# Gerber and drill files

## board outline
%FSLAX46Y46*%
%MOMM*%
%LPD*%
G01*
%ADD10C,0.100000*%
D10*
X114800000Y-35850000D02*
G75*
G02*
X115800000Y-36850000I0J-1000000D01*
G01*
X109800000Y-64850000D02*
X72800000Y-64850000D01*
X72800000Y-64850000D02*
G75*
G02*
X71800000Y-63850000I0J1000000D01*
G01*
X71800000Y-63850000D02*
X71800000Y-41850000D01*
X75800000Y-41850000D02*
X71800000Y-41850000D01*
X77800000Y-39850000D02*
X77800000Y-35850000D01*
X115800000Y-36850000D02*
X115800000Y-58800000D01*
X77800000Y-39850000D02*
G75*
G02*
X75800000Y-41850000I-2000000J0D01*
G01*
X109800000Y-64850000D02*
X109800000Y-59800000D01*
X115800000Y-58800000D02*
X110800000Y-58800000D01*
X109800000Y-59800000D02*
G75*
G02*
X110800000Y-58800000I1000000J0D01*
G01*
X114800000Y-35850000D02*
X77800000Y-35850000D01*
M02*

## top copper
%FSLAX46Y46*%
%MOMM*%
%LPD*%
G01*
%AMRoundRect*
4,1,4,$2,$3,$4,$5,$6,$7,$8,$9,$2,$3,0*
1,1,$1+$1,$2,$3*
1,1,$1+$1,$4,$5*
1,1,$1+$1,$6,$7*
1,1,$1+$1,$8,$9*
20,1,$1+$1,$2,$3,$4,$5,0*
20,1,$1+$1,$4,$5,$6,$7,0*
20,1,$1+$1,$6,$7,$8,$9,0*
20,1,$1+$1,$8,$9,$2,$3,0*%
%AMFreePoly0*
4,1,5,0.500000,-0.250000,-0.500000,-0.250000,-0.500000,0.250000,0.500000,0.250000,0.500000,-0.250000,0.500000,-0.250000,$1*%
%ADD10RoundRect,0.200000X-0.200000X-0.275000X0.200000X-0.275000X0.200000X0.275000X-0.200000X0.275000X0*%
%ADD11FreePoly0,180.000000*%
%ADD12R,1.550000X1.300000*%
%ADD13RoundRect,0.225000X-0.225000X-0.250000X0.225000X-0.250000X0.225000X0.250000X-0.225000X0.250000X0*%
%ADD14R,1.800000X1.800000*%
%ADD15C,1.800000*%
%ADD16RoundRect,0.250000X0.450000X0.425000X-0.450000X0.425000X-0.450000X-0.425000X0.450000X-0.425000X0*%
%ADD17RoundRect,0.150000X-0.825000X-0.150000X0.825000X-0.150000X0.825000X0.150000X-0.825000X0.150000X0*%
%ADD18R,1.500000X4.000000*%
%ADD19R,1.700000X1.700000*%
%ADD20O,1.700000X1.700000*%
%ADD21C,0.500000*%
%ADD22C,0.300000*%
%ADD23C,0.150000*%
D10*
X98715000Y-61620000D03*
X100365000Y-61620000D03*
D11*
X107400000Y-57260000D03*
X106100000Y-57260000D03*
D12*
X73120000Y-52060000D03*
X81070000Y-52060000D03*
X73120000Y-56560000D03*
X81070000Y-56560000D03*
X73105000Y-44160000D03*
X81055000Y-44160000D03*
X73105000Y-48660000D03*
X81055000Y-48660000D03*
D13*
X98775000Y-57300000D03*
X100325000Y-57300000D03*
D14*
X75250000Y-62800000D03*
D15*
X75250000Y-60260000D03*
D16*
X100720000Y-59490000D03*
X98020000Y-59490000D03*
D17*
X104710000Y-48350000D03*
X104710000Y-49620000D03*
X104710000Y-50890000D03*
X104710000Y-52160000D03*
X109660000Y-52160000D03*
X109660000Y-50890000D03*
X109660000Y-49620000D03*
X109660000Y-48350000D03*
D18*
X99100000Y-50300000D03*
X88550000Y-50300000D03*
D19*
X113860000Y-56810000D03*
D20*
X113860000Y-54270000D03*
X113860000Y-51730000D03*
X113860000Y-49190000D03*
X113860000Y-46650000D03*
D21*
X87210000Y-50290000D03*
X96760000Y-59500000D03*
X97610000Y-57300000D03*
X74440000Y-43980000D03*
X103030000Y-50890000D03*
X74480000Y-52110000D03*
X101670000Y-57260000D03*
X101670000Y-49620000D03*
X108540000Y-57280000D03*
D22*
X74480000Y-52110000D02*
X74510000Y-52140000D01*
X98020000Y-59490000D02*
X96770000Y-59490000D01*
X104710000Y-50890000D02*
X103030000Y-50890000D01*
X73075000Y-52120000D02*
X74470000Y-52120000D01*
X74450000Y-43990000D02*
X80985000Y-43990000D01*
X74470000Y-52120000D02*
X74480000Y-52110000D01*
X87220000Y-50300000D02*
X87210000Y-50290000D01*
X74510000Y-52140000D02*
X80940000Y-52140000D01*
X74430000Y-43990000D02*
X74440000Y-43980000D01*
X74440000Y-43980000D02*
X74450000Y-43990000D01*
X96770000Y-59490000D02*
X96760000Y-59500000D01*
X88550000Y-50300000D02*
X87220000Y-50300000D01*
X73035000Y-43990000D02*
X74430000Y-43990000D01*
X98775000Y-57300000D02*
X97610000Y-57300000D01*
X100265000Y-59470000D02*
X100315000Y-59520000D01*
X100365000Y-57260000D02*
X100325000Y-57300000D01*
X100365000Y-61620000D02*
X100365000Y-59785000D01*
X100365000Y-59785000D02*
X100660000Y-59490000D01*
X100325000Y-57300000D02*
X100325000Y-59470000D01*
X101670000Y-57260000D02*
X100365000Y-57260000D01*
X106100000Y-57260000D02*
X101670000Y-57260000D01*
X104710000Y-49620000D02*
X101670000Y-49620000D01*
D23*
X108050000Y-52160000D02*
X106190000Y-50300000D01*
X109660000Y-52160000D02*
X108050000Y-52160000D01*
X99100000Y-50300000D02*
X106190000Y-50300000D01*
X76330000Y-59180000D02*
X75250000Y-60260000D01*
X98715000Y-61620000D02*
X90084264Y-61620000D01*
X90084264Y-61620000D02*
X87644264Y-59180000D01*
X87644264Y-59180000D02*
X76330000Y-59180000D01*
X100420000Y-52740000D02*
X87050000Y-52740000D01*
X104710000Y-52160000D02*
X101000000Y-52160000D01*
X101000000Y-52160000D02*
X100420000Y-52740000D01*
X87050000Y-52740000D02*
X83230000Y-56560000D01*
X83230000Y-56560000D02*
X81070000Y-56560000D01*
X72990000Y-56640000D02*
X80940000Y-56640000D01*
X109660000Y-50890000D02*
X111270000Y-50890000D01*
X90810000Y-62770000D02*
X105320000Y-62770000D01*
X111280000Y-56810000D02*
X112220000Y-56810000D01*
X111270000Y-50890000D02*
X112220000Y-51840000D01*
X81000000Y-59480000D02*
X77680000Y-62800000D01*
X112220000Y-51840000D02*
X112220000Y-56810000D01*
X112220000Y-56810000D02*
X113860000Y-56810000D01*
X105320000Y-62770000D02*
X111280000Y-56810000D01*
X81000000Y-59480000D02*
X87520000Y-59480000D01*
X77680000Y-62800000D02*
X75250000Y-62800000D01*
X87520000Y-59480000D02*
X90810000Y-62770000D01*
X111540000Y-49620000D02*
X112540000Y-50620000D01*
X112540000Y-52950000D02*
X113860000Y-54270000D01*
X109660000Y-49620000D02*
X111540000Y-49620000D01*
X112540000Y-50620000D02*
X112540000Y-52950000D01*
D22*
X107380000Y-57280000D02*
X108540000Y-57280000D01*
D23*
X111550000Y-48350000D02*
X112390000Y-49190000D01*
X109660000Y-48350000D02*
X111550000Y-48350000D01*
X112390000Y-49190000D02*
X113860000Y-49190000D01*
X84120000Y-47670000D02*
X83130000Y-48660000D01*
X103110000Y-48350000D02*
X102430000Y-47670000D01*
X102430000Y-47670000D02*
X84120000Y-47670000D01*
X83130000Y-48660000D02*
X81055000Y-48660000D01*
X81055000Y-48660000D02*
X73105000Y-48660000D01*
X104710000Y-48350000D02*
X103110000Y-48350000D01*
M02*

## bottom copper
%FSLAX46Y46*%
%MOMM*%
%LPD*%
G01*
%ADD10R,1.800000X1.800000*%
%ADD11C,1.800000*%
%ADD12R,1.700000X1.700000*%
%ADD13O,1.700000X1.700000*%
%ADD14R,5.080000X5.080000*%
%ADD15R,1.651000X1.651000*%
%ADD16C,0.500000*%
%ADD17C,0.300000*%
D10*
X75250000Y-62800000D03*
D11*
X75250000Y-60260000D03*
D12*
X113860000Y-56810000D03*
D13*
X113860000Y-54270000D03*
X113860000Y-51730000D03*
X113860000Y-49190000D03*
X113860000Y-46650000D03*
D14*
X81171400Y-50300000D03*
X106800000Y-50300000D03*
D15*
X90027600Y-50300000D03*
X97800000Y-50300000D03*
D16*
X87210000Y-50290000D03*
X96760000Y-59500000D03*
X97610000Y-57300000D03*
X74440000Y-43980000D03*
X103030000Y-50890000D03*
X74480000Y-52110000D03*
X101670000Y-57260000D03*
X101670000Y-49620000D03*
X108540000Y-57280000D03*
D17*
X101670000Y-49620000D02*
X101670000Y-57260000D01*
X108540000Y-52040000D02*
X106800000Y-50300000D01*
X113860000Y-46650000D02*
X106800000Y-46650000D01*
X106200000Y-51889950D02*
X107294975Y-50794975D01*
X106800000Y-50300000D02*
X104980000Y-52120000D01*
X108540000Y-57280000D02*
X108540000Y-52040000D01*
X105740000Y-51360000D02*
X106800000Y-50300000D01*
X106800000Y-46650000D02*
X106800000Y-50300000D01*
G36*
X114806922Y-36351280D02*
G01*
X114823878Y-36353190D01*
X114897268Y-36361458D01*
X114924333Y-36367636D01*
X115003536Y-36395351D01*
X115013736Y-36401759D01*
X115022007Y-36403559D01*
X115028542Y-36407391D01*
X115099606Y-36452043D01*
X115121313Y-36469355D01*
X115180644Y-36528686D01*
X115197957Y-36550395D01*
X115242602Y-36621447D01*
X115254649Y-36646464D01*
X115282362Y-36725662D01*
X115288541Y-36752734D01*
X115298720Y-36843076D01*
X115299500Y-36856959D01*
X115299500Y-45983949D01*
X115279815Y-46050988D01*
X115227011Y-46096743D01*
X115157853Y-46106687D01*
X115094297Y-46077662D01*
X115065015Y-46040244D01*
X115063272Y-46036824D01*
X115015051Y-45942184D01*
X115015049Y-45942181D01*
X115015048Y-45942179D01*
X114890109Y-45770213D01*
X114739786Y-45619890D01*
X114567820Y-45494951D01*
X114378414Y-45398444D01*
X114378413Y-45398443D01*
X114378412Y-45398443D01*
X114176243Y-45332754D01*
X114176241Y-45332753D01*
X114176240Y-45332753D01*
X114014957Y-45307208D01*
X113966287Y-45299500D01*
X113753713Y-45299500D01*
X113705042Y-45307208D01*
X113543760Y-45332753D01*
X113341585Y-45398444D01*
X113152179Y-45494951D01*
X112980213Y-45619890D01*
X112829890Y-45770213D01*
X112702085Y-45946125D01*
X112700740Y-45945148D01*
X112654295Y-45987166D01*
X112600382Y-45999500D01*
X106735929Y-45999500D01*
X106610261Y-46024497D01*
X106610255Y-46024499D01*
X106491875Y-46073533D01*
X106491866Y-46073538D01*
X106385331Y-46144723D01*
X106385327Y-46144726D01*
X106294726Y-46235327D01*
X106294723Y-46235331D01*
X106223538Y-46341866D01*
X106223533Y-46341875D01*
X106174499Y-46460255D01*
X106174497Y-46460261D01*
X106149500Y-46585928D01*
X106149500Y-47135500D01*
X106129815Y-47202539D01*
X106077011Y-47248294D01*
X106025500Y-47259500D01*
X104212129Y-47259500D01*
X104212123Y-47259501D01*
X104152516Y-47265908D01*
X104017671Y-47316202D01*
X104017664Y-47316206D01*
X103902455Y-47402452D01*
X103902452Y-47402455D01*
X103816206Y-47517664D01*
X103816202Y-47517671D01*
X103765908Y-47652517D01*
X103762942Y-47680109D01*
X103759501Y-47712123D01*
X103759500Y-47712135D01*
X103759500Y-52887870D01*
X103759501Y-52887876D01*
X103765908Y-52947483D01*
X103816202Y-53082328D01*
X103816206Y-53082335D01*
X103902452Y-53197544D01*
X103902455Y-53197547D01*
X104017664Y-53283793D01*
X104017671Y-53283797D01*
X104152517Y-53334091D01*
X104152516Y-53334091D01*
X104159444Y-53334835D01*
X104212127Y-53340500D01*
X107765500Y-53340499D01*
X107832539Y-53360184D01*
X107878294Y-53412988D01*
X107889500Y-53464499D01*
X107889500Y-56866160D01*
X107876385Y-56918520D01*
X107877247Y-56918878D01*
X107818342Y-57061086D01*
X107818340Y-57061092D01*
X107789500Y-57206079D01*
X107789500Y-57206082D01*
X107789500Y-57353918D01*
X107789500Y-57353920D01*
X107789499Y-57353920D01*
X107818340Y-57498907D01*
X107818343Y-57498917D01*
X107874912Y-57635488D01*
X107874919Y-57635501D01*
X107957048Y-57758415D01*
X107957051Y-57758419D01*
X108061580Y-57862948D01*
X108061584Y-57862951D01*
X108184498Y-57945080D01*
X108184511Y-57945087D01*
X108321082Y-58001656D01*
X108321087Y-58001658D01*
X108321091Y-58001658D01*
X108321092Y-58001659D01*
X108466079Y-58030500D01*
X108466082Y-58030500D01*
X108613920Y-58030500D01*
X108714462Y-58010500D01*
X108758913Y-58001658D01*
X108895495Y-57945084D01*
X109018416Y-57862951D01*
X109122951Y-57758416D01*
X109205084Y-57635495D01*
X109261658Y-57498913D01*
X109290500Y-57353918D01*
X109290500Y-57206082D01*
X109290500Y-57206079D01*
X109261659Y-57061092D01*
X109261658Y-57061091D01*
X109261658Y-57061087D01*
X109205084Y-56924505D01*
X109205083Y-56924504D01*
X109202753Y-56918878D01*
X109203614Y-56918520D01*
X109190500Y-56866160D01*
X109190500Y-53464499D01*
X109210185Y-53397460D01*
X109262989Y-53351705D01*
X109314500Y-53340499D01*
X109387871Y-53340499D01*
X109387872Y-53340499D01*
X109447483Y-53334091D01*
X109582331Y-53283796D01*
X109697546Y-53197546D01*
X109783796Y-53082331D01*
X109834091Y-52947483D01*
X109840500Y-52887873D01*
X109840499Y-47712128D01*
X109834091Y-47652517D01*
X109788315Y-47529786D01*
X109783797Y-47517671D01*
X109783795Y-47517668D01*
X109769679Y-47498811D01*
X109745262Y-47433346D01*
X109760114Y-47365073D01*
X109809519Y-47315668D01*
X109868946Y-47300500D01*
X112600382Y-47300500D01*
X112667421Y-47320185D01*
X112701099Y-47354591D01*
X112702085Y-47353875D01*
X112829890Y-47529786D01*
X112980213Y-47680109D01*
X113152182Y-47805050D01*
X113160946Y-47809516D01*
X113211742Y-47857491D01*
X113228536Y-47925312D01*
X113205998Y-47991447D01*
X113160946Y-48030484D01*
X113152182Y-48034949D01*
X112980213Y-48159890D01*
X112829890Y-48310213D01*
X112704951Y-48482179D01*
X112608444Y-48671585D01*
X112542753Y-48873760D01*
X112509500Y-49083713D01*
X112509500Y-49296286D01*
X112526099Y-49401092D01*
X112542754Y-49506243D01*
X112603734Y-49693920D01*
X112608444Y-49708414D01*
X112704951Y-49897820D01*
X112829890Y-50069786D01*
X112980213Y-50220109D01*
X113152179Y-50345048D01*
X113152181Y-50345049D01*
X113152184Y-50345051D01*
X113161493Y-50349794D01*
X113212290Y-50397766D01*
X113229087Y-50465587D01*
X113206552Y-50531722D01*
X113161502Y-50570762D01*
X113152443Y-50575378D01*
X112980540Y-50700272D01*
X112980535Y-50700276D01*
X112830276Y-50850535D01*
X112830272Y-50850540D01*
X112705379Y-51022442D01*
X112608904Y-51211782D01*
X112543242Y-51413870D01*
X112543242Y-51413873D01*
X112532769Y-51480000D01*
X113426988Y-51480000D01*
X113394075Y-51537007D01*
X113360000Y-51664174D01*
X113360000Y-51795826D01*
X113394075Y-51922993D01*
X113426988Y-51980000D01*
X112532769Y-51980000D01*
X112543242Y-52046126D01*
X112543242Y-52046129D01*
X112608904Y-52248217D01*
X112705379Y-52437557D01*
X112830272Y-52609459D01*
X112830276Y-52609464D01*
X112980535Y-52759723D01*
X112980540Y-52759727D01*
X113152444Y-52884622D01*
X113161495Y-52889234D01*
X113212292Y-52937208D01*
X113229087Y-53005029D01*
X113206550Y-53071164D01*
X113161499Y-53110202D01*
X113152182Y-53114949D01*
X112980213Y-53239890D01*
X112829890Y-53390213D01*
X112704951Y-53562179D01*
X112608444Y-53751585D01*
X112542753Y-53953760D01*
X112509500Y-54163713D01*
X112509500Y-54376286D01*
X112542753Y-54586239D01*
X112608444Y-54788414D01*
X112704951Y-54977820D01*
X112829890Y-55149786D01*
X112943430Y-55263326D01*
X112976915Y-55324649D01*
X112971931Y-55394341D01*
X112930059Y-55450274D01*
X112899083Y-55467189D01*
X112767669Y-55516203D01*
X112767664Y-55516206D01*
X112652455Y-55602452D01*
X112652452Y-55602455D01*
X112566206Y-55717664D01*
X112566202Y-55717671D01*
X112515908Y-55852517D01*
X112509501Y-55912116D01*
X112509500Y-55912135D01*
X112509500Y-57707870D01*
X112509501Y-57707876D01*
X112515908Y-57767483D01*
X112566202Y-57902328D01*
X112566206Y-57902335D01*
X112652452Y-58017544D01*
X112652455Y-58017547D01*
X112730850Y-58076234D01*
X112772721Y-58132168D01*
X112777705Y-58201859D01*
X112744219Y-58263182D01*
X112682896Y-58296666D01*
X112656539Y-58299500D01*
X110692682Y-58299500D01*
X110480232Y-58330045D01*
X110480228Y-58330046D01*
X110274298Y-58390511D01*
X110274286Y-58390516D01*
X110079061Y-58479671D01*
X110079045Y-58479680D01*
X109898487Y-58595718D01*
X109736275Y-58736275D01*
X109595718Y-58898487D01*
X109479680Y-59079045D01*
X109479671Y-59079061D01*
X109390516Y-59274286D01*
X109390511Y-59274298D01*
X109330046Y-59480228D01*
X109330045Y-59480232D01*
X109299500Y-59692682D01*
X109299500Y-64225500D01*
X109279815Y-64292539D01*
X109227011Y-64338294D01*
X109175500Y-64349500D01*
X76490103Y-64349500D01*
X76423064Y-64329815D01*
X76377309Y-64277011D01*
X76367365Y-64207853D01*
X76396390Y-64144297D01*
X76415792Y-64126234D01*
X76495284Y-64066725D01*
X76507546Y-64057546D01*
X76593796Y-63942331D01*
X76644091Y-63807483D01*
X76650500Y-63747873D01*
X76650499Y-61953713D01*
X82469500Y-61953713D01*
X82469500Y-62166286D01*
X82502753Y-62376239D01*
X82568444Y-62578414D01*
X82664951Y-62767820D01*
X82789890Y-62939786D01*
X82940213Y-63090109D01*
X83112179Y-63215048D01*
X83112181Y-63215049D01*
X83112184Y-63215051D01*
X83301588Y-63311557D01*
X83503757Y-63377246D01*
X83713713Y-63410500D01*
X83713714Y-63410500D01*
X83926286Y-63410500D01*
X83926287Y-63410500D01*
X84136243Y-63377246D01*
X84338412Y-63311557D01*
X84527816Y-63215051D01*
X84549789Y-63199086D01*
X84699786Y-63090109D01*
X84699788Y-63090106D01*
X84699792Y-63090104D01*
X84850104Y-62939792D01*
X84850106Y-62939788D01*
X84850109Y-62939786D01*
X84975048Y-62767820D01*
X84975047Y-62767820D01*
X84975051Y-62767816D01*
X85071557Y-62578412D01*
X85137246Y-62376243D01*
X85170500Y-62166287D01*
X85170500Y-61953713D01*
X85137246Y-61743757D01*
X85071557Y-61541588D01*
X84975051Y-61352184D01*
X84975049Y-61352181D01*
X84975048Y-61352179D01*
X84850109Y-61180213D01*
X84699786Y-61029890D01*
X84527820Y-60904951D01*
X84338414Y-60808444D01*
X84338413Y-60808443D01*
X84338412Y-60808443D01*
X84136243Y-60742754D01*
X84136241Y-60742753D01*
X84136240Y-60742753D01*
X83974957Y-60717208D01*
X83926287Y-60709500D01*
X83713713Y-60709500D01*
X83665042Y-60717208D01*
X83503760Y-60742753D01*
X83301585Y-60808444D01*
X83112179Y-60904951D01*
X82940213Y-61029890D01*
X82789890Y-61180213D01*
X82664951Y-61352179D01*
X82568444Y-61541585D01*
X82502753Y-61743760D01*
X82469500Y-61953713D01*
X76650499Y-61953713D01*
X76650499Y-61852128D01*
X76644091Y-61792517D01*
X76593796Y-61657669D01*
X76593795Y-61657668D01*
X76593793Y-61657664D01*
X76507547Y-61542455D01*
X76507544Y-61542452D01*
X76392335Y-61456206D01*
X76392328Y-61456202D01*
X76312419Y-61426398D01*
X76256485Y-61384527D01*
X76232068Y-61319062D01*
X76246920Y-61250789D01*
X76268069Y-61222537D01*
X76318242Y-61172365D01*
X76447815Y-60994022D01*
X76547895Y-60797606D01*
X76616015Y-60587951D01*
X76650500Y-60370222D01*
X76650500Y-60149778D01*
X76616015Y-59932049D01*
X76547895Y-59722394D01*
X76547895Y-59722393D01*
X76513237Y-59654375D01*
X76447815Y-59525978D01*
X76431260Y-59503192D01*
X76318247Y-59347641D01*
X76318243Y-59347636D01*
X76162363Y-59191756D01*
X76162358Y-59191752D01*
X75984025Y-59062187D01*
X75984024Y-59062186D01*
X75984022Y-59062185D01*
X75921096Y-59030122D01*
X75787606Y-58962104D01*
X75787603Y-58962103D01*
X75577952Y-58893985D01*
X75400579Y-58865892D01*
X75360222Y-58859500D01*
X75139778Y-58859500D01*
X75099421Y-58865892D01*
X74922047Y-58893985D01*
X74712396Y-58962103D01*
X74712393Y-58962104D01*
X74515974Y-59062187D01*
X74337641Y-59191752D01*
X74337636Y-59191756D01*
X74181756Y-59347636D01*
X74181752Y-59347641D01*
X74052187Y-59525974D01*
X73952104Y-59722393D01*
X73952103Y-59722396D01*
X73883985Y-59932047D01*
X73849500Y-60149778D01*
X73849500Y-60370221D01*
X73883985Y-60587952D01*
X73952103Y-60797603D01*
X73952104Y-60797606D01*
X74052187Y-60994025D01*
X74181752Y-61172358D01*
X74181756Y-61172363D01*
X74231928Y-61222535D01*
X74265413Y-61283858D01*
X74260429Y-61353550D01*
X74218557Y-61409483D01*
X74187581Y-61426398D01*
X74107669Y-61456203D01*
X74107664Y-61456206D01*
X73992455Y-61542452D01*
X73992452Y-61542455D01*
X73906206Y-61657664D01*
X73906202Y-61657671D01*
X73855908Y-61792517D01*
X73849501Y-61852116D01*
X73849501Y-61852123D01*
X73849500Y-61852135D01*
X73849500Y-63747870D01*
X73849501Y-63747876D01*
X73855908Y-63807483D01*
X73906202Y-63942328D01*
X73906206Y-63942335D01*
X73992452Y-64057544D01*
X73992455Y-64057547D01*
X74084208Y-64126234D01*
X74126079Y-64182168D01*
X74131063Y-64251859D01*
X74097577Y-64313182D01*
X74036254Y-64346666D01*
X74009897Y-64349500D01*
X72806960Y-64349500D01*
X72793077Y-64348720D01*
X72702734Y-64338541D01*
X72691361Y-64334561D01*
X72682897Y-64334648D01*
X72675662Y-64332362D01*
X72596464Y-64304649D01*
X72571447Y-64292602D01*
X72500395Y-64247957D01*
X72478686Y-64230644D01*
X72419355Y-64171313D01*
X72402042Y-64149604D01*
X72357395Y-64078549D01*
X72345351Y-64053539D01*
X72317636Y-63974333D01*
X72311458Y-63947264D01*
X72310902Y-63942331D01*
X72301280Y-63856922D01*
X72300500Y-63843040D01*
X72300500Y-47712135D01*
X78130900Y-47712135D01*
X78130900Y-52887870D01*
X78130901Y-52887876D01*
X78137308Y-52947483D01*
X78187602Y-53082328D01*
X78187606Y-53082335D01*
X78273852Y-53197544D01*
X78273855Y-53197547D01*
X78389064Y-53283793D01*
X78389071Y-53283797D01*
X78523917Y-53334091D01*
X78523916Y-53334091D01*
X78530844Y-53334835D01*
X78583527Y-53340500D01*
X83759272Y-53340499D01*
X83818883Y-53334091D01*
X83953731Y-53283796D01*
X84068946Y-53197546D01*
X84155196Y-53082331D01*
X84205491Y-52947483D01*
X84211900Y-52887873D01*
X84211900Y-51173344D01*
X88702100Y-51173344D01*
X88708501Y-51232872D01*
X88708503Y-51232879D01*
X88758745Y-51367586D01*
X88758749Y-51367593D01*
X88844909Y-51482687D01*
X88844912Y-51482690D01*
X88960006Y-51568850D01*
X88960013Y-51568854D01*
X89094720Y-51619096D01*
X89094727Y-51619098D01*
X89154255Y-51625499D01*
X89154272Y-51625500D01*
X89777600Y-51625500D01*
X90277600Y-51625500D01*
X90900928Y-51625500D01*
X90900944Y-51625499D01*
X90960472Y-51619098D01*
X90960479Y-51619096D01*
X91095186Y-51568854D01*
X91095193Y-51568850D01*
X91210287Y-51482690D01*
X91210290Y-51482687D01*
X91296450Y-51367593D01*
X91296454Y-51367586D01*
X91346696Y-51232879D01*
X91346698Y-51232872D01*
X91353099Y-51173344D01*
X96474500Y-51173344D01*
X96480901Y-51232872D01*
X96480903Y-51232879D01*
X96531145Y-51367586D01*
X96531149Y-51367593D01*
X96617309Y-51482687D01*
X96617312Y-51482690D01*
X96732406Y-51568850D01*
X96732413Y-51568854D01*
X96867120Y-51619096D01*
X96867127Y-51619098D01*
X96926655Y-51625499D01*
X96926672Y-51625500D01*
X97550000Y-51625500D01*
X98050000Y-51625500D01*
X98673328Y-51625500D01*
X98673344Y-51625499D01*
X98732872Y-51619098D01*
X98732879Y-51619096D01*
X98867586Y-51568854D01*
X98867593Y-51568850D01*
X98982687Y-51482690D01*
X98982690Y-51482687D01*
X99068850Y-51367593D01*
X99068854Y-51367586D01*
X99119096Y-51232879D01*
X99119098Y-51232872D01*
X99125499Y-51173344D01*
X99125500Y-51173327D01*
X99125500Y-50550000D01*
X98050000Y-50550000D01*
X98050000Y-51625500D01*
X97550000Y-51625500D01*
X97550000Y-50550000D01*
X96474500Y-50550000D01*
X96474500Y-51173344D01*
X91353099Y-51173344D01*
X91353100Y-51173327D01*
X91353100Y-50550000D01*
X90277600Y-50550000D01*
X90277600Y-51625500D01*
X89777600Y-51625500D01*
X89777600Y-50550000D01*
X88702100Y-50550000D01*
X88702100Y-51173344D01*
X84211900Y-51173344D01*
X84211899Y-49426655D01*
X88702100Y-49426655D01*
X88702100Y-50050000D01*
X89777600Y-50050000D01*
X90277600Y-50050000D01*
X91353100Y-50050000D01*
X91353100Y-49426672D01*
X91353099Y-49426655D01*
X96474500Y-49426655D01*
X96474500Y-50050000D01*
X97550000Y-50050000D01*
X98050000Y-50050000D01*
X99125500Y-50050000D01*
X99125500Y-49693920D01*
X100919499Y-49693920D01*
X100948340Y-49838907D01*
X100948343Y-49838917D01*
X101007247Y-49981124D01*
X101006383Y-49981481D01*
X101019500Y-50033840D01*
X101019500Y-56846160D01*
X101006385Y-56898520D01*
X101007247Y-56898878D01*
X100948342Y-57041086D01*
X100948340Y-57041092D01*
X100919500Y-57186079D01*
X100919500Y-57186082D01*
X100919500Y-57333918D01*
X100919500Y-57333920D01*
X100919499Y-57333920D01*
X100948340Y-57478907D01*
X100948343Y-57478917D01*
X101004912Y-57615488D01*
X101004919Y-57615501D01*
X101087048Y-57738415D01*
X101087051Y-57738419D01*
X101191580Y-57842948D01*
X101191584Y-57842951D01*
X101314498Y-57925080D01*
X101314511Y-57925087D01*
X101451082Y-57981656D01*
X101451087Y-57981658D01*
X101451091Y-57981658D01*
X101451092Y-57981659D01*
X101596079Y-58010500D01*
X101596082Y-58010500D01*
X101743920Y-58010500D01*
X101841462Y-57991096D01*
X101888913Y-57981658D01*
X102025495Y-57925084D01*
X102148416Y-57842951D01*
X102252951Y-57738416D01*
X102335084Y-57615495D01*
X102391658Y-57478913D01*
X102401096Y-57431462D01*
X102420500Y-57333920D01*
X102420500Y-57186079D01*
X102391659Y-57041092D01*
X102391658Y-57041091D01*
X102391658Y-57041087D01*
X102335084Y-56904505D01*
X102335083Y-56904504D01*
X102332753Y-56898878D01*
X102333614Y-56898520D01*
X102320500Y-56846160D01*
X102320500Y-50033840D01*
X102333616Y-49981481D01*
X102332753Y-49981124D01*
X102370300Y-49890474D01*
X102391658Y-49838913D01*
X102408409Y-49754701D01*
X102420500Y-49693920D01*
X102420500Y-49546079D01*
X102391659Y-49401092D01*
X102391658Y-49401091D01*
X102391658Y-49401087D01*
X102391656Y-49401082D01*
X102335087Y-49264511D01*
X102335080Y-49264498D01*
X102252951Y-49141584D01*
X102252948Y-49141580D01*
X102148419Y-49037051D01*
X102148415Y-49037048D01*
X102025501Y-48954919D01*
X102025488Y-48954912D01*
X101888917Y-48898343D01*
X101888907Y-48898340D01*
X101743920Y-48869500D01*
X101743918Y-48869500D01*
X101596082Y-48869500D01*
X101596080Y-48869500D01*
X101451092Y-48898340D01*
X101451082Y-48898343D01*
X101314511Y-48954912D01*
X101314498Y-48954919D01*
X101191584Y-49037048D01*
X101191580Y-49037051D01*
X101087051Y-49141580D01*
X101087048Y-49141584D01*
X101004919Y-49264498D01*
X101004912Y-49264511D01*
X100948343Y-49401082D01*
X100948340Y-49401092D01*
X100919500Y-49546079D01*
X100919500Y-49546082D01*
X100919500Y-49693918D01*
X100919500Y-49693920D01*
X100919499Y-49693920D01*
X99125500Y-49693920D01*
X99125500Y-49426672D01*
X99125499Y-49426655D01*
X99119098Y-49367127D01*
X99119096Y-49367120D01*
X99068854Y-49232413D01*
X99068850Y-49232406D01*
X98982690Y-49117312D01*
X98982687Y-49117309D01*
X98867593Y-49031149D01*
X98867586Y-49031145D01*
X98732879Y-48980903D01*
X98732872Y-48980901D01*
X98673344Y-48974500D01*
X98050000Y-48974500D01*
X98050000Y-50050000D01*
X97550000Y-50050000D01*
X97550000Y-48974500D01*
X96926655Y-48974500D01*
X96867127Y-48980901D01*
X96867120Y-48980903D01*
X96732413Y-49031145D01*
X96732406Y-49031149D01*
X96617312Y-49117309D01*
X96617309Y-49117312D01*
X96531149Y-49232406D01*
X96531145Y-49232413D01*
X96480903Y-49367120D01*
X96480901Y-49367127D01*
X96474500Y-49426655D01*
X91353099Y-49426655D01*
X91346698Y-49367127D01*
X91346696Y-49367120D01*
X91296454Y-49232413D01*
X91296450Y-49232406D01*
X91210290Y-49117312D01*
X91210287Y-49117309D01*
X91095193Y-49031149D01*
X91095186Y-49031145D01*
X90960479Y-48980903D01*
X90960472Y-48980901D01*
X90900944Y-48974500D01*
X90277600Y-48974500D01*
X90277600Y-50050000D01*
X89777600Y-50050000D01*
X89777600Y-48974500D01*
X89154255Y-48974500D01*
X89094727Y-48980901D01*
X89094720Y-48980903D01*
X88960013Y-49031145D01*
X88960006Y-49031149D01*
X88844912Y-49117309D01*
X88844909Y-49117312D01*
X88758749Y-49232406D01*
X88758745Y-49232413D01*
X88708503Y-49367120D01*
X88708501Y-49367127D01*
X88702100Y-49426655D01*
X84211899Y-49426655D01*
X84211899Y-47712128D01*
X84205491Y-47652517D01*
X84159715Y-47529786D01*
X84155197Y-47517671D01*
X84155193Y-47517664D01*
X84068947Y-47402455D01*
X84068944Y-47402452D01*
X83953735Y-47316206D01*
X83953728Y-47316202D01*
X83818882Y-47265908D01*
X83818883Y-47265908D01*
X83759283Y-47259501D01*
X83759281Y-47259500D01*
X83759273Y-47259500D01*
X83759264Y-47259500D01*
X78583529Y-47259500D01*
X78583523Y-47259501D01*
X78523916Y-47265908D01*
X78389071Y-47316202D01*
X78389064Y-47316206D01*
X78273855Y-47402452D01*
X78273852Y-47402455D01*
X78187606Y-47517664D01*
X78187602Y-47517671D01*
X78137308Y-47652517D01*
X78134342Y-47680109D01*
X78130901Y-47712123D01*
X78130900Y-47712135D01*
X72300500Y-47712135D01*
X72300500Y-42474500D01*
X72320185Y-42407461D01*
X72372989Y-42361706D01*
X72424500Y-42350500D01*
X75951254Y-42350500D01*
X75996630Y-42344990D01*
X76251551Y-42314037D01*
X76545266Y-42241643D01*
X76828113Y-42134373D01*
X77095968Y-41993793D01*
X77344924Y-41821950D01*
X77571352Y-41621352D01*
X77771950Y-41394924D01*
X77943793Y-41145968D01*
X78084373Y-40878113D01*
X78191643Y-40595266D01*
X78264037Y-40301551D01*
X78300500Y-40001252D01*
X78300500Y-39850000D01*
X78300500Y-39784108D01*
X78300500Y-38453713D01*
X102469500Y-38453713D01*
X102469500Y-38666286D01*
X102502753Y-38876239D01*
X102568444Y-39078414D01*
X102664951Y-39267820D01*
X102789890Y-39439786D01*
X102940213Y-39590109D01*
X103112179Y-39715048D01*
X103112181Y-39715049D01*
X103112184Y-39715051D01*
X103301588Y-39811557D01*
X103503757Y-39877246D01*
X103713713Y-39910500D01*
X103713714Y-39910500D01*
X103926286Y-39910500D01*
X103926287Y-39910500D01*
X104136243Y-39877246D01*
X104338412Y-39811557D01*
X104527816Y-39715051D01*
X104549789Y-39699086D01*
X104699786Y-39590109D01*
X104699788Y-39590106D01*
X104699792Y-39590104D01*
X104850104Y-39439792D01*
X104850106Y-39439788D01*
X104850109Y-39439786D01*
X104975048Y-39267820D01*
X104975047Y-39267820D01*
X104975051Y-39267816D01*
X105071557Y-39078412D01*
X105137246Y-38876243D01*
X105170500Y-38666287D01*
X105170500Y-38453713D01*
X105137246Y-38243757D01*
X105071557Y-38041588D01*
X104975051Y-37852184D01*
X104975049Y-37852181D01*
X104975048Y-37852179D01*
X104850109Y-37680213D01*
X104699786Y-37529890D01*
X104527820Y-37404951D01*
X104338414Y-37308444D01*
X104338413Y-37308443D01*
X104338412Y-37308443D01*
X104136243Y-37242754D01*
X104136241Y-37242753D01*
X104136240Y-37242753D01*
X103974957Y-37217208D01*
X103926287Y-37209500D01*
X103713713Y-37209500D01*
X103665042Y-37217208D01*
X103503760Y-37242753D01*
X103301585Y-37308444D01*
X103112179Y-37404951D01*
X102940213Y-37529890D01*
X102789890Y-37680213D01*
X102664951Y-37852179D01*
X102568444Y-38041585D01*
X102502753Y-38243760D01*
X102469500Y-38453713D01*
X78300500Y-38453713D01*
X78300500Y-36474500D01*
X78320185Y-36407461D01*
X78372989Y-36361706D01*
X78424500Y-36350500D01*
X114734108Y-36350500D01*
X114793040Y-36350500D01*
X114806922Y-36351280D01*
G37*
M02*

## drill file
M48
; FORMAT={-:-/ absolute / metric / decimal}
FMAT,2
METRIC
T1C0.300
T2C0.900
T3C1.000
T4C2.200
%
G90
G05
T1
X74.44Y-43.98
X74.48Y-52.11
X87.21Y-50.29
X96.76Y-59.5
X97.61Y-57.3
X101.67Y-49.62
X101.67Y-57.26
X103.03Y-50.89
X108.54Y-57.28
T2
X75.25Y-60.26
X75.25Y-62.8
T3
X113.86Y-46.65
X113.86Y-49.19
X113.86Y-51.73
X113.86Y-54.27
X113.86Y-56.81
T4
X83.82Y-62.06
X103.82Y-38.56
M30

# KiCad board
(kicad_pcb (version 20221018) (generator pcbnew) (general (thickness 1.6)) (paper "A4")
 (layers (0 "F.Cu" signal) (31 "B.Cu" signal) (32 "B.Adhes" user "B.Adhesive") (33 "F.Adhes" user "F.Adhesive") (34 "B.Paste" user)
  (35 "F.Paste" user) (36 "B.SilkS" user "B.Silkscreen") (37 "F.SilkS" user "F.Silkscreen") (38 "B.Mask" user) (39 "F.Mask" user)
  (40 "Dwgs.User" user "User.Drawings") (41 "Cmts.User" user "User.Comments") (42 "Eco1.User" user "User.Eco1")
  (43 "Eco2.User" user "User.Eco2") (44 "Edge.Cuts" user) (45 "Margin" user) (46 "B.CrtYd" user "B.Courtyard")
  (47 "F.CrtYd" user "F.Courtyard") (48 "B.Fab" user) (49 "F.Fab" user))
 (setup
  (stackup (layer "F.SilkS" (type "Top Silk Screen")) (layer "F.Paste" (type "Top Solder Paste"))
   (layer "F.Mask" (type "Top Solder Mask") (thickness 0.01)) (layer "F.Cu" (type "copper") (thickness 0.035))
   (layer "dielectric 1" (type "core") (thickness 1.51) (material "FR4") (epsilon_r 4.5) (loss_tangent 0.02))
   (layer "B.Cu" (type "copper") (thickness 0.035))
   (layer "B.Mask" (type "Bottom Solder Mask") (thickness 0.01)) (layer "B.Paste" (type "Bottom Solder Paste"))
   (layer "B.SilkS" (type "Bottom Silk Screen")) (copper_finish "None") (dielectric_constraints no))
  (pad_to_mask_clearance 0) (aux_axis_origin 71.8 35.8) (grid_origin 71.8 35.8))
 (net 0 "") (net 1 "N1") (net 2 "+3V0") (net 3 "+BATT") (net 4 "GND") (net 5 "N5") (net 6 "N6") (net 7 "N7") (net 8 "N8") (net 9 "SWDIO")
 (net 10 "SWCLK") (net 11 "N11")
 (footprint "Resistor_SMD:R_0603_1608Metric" (layer "F.Cu") (at 99.54 61.62)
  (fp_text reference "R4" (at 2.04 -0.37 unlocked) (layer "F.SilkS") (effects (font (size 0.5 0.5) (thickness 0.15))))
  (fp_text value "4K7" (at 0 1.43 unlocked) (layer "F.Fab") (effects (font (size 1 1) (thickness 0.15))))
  (pad "1" smd roundrect (at -0.825 0) (size 0.8 0.95) (layers "F.Cu" "F.Paste" "F.Mask") (roundrect_rratio 0.25) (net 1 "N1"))
  (pad "2" smd roundrect (at 0.825 0) (size 0.8 0.95) (layers "F.Cu" "F.Paste" "F.Mask") (roundrect_rratio 0.25) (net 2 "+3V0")))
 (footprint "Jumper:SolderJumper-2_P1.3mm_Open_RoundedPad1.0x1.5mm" (layer "F.Cu") (at 106.75 57.26 180) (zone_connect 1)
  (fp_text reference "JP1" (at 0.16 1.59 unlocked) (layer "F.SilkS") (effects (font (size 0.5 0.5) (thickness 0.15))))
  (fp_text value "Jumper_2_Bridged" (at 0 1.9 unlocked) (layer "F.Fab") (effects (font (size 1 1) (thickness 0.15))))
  (pad "1" smd custom (at -0.65 0 180) (size 1 0.5) (layers "F.Cu" "F.Mask") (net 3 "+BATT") (zone_connect 2) (thermal_bridge_angle 45)
   (options (clearance outline) (anchor rect)) (primitives))
  (pad "2" smd custom (at 0.65 0 180) (size 1 0.5) (layers "F.Cu" "F.Mask") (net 2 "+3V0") (zone_connect 2) (thermal_bridge_angle 45)
   (options (clearance outline) (anchor rect)) (primitives)))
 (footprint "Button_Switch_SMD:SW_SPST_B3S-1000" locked (layer "F.Cu") (at 77.095 54.31)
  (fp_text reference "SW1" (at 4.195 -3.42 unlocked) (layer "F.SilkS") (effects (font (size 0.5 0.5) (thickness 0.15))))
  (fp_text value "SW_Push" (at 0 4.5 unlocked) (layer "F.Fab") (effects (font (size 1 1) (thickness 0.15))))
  (pad "1" smd rect locked (at -3.975 -2.25) (size 1.55 1.3) (layers "F.Cu" "F.Paste" "F.Mask") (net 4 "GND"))
  (pad "1" smd rect locked (at 3.975 -2.25) (size 1.55 1.3) (layers "F.Cu" "F.Paste" "F.Mask") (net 4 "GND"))
  (pad "2" smd rect locked (at -3.975 2.25) (size 1.55 1.3) (layers "F.Cu" "F.Paste" "F.Mask") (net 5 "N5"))
  (pad "2" smd rect locked (at 3.975 2.25) (size 1.55 1.3) (layers "F.Cu" "F.Paste" "F.Mask") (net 5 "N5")))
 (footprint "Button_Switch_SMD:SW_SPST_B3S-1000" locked (layer "F.Cu") (at 77.08 46.41)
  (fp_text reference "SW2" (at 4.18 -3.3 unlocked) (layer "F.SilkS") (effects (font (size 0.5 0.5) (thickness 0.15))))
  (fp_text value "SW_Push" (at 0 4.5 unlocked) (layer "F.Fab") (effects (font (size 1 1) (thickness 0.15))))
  (pad "1" smd rect locked (at -3.975 -2.25) (size 1.55 1.3) (layers "F.Cu" "F.Paste" "F.Mask") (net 4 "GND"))
  (pad "1" smd rect locked (at 3.975 -2.25) (size 1.55 1.3) (layers "F.Cu" "F.Paste" "F.Mask") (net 4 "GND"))
  (pad "2" smd rect locked (at -3.975 2.25) (size 1.55 1.3) (layers "F.Cu" "F.Paste" "F.Mask") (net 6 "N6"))
  (pad "2" smd rect locked (at 3.975 2.25) (size 1.55 1.3) (layers "F.Cu" "F.Paste" "F.Mask") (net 6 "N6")))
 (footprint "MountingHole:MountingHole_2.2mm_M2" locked (layer "F.Cu") (at 103.82 38.56)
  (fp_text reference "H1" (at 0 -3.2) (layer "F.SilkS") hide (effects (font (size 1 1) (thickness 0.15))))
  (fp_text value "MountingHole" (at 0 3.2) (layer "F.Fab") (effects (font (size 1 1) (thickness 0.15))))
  (pad "" np_thru_hole circle locked (at 0 0) (size 2.2 2.2) (drill 2.2) (layers "*.Cu" "*.Mask")))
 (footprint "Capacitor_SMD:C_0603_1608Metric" (layer "F.Cu") (at 99.55 57.3)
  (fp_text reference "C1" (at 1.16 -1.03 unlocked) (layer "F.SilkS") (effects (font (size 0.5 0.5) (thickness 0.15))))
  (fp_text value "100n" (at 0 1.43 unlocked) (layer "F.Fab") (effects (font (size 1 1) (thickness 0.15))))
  (pad "1" smd roundrect (at -0.775 0) (size 0.9 0.95) (layers "F.Cu" "F.Paste" "F.Mask") (roundrect_rratio 0.25) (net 4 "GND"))
  (pad "2" smd roundrect (at 0.775 0) (size 0.9 0.95) (layers "F.Cu" "F.Paste" "F.Mask") (roundrect_rratio 0.25) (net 2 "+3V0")))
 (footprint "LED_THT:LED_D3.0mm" (layer "F.Cu") (at 75.25 62.8 90)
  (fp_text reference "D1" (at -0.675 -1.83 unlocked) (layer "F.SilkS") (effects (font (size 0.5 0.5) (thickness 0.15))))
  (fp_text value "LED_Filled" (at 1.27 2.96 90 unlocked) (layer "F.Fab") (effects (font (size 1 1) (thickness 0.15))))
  (pad "1" thru_hole rect (at 0 0 90) (size 1.8 1.8) (drill 0.9) (layers "*.Cu" "*.Mask") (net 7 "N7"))
  (pad "2" thru_hole circle (at 2.54 0 90) (size 1.8 1.8) (drill 0.9) (layers "*.Cu" "*.Mask") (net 1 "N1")))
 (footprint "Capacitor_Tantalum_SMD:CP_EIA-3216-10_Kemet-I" (layer "F.Cu") (at 99.37 59.49 180)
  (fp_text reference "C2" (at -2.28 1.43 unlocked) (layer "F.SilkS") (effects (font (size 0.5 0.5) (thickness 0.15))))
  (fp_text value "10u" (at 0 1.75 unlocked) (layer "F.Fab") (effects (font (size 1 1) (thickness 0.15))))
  (pad "1" smd roundrect (at -1.35 0 180) (size 1.4 1.35) (layers "F.Cu" "F.Paste" "F.Mask") (roundrect_rratio 0.185185) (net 2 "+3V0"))
  (pad "2" smd roundrect (at 1.35 0 180) (size 1.4 1.35) (layers "F.Cu" "F.Paste" "F.Mask") (roundrect_rratio 0.185185) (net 4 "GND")))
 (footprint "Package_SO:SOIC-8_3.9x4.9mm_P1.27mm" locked (layer "F.Cu") (at 107.185 50.255)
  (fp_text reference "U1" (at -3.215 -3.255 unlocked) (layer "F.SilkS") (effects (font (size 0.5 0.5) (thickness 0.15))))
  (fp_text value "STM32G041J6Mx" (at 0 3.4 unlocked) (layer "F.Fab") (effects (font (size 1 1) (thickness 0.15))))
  (pad "1" smd roundrect locked (at -2.475 -1.905) (size 1.95 0.6) (layers "F.Cu" "F.Paste" "F.Mask") (roundrect_rratio 0.25) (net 6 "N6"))
  (pad "2" smd roundrect locked (at -2.475 -0.635) (size 1.95 0.6) (layers "F.Cu" "F.Paste" "F.Mask") (roundrect_rratio 0.25) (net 2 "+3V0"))
  (pad "3" smd roundrect locked (at -2.475 0.635) (size 1.95 0.6) (layers "F.Cu" "F.Paste" "F.Mask") (roundrect_rratio 0.25) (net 4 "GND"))
  (pad "4" smd roundrect locked (at -2.475 1.905) (size 1.95 0.6) (layers "F.Cu" "F.Paste" "F.Mask") (roundrect_rratio 0.25) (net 5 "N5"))
  (pad "5" smd roundrect locked (at 2.475 1.905) (size 1.95 0.6) (layers "F.Cu" "F.Paste" "F.Mask") (roundrect_rratio 0.25) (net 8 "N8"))
  (pad "6" smd roundrect locked (at 2.475 0.635) (size 1.95 0.6) (layers "F.Cu" "F.Paste" "F.Mask") (roundrect_rratio 0.25) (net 7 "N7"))
  (pad "7" smd roundrect locked (at 2.475 -0.635) (size 1.95 0.6) (layers "F.Cu" "F.Paste" "F.Mask") (roundrect_rratio 0.25) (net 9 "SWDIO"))
  (pad "8" smd roundrect locked (at 2.475 -1.905) (size 1.95 0.6) (layers "F.Cu" "F.Paste" "F.Mask") (roundrect_rratio 0.25)
   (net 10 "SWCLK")))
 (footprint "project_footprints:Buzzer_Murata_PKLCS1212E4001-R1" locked (layer "F.Cu") (at 93.8 50.3 180)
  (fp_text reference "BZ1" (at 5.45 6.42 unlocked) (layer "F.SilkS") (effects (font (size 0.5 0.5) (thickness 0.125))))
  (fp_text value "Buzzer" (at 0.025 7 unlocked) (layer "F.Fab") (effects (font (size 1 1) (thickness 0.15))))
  (pad "1" smd rect locked (at -5.3 0 180) (size 1.5 4) (layers "F.Cu" "F.Paste" "F.Mask") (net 8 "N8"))
  (pad "2" smd rect locked (at 5.25 0 180) (size 1.5 4) (layers "F.Cu" "F.Paste" "F.Mask") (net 4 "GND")))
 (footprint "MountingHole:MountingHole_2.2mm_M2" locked (layer "F.Cu") (at 83.82 62.06)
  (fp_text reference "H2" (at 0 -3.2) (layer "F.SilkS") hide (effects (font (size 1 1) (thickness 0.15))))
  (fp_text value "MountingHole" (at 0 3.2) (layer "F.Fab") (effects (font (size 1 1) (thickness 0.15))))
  (pad "" np_thru_hole circle locked (at 0 0) (size 2.2 2.2) (drill 2.2) (layers "*.Cu" "*.Mask")))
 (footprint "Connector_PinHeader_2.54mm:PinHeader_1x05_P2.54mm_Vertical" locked (layer "B.Cu") (at 113.86 56.81)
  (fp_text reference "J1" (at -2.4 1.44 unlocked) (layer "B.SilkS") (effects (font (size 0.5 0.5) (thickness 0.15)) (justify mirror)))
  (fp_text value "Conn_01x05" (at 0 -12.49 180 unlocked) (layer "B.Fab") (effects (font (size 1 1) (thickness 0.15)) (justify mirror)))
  (pad "1" thru_hole rect locked (at 0 0) (size 1.7 1.7) (drill 1) (layers "*.Cu" "*.Mask") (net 7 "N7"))
  (pad "2" thru_hole oval locked (at 0 -2.54) (size 1.7 1.7) (drill 1) (layers "*.Cu" "*.Mask") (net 9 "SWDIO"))
  (pad "3" thru_hole oval locked (at 0 -5.08) (size 1.7 1.7) (drill 1) (layers "*.Cu" "*.Mask") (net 4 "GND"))
  (pad "4" thru_hole oval locked (at 0 -7.62) (size 1.7 1.7) (drill 1) (layers "*.Cu" "*.Mask") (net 10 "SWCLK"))
  (pad "5" thru_hole oval locked (at 0 -10.16) (size 1.7 1.7) (drill 1) (layers "*.Cu" "*.Mask") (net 3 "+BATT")))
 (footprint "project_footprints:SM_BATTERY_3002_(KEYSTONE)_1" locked (layer "B.Cu") (at 93.973 50.3 180)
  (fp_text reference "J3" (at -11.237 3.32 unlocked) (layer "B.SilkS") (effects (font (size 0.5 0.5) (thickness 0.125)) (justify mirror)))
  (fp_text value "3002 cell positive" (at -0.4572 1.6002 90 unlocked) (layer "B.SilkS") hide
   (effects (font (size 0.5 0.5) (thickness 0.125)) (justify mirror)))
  (pad "1" smd rect locked (at 12.8016 0 90) (size 5.08 5.08) (layers "B.Cu" "B.Paste" "B.Mask") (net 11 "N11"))
  (pad "2" smd rect locked (at -12.827 0 90) (size 5.08 5.08) (layers "B.Cu" "B.Paste" "B.Mask") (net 3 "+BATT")))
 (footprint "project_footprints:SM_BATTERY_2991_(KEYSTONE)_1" (layer "B.Cu") (at 93.9138 50.3 180)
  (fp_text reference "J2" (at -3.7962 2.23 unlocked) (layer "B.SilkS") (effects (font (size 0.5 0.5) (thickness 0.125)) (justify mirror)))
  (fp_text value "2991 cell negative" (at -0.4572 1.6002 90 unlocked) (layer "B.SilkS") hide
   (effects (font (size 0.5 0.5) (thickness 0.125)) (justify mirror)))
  (pad "1" smd rect (at 3.8862 0 90) (size 1.651 1.651) (layers "B.Cu" "B.Paste" "B.Mask") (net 4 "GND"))
  (pad "2" smd rect (at -3.8862 0 90) (size 1.651 1.651) (layers "B.Cu" "B.Paste" "B.Mask") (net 4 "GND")))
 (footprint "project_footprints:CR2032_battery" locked (layer "B.Cu") (at 93.9138 50.3 180)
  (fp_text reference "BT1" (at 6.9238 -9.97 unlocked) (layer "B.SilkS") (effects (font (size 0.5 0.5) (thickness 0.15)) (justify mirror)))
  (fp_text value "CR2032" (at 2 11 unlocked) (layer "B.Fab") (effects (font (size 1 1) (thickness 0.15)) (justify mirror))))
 (gr_arc (start 114.8 35.85) (mid 115.507107 36.142893) (end 115.8 36.85) (stroke (width 0.1) (type solid)) (layer "Edge.Cuts"))
 (gr_line (start 109.8 64.85) (end 72.8 64.85) (stroke (width 0.1) (type solid)) (layer "Edge.Cuts"))
 (gr_arc (start 72.8 64.85) (mid 72.092893 64.557107) (end 71.8 63.85) (stroke (width 0.1) (type solid)) (layer "Edge.Cuts"))
 (gr_line (start 71.8 63.85) (end 71.8 41.85) (stroke (width 0.1) (type solid)) (layer "Edge.Cuts"))
 (gr_line (start 75.8 41.85) (end 71.8 41.85) (stroke (width 0.1) (type solid)) (layer "Edge.Cuts"))
 (gr_line (start 77.8 39.85) (end 77.8 35.85) (stroke (width 0.1) (type solid)) (layer "Edge.Cuts"))
 (gr_line (start 115.8 36.85) (end 115.8 58.8) (stroke (width 0.1) (type solid)) (layer "Edge.Cuts"))
 (gr_arc (start 77.8 39.85) (mid 77.214214 41.264214) (end 75.8 41.85) (stroke (width 0.1) (type solid)) (layer "Edge.Cuts"))
 (gr_line (start 109.8 64.85) (end 109.8 59.8) (stroke (width 0.1) (type solid)) (layer "Edge.Cuts"))
 (gr_line (start 115.8 58.8) (end 110.8 58.8) (stroke (width 0.1) (type solid)) (layer "Edge.Cuts"))
 (gr_arc (start 109.8 59.8) (mid 110.092893 59.092893) (end 110.8 58.8) (stroke (width 0.1) (type solid)) (layer "Edge.Cuts"))
 (gr_line (start 114.8 35.85) (end 77.8 35.85) (stroke (width 0.1) (type solid)) (layer "Edge.Cuts"))
 (segment (start 74.48 52.11) (end 74.51 52.14) (width 0.3) (layer "F.Cu") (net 4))
 (segment (start 98.02 59.49) (end 96.77 59.49) (width 0.3) (layer "F.Cu") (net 4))
 (segment (start 104.71 50.89) (end 103.03 50.89) (width 0.3) (layer "F.Cu") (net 4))
 (segment (start 73.075 52.12) (end 74.47 52.12) (width 0.3) (layer "F.Cu") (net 4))
 (segment (start 74.45 43.99) (end 80.985 43.99) (width 0.3) (layer "F.Cu") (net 4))
 (segment (start 74.47 52.12) (end 74.48 52.11) (width 0.3) (layer "F.Cu") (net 4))
 (segment (start 87.22 50.3) (end 87.21 50.29) (width 0.3) (layer "F.Cu") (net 4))
 (segment (start 74.51 52.14) (end 80.94 52.14) (width 0.3) (layer "F.Cu") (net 4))
 (segment (start 74.43 43.99) (end 74.44 43.98) (width 0.3) (layer "F.Cu") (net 4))
 (segment (start 74.44 43.98) (end 74.45 43.99) (width 0.3) (layer "F.Cu") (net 4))
 (segment (start 96.77 59.49) (end 96.76 59.5) (width 0.3) (layer "F.Cu") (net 4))
 (segment (start 88.55 50.3) (end 87.22 50.3) (width 0.3) (layer "F.Cu") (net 4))
 (segment (start 73.035 43.99) (end 74.43 43.99) (width 0.3) (layer "F.Cu") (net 4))
 (segment (start 98.775 57.3) (end 97.61 57.3) (width 0.3) (layer "F.Cu") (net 4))
 (via (at 87.21 50.29) (size 0.5) (drill 0.3) (layers "F.Cu" "B.Cu") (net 4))
 (via (at 96.76 59.5) (size 0.5) (drill 0.3) (layers "F.Cu" "B.Cu") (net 4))
 (via (at 97.61 57.3) (size 0.5) (drill 0.3) (layers "F.Cu" "B.Cu") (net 4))
 (via (at 74.44 43.98) (size 0.5) (drill 0.3) (layers "F.Cu" "B.Cu") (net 4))
 (via (at 103.03 50.89) (size 0.5) (drill 0.3) (layers "F.Cu" "B.Cu") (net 4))
 (via (at 74.48 52.11) (size 0.5) (drill 0.3) (layers "F.Cu" "B.Cu") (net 4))
 (segment (start 100.265 59.47) (end 100.315 59.52) (width 0.3) (layer "F.Cu") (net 2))
 (segment (start 100.365 57.26) (end 100.325 57.3) (width 0.3) (layer "F.Cu") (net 2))
 (segment (start 100.365 61.62) (end 100.365 59.785) (width 0.3) (layer "F.Cu") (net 2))
 (segment (start 100.365 59.785) (end 100.66 59.49) (width 0.3) (layer "F.Cu") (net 2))
 (segment (start 100.325 57.3) (end 100.325 59.47) (width 0.3) (layer "F.Cu") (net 2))
 (segment (start 101.67 57.26) (end 100.365 57.26) (width 0.3) (layer "F.Cu") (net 2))
 (segment (start 106.1 57.26) (end 101.67 57.26) (width 0.3) (layer "F.Cu") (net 2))
 (segment (start 104.71 49.62) (end 101.67 49.62) (width 0.3) (layer "F.Cu") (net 2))
 (via (at 101.67 57.26) (size 0.5) (drill 0.3) (layers "F.Cu" "B.Cu") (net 2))
 (via (at 101.67 49.62) (size 0.5) (drill 0.3) (layers "F.Cu" "B.Cu") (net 2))
 (segment (start 101.67 49.62) (end 101.67 57.26) (width 0.3) (layer "B.Cu") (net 2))
 (segment (start 108.05 52.16) (end 106.19 50.3) (width 0.15) (layer "F.Cu") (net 8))
 (segment (start 109.66 52.16) (end 108.05 52.16) (width 0.15) (layer "F.Cu") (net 8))
 (segment (start 99.1 50.3) (end 106.19 50.3) (width 0.15) (layer "F.Cu") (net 8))
 (segment (start 76.33 59.18) (end 75.25 60.26) (width 0.15) (layer "F.Cu") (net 1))
 (segment (start 98.715 61.62) (end 90.084264 61.62) (width 0.15) (layer "F.Cu") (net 1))
 (segment (start 90.084264 61.62) (end 87.644264 59.18) (width 0.15) (layer "F.Cu") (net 1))
 (segment (start 87.644264 59.18) (end 76.33 59.18) (width 0.15) (layer "F.Cu") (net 1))
 (segment (start 100.42 52.74) (end 87.05 52.74) (width 0.15) (layer "F.Cu") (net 5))
 (segment (start 104.71 52.16) (end 101 52.16) (width 0.15) (layer "F.Cu") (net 5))
 (segment (start 101 52.16) (end 100.42 52.74) (width 0.15) (layer "F.Cu") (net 5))
 (segment (start 87.05 52.74) (end 83.23 56.56) (width 0.15) (layer "F.Cu") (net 5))
 (segment (start 83.23 56.56) (end 81.07 56.56) (width 0.15) (layer "F.Cu") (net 5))
 (segment (start 72.99 56.64) (end 80.94 56.64) (width 0.15) (layer "F.Cu") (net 5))
 (segment (start 109.66 50.89) (end 111.27 50.89) (width 0.15) (layer "F.Cu") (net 7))
 (segment (start 90.81 62.77) (end 105.32 62.77) (width 0.15) (layer "F.Cu") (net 7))
 (segment (start 111.28 56.81) (end 112.22 56.81) (width 0.15) (layer "F.Cu") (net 7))
 (segment (start 111.27 50.89) (end 112.22 51.84) (width 0.15) (layer "F.Cu") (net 7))
 (segment (start 81 59.48) (end 77.68 62.8) (width 0.15) (layer "F.Cu") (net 7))
 (segment (start 112.22 51.84) (end 112.22 56.81) (width 0.15) (layer "F.Cu") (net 7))
 (segment (start 112.22 56.81) (end 113.86 56.81) (width 0.15) (layer "F.Cu") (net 7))
 (segment (start 105.32 62.77) (end 111.28 56.81) (width 0.15) (layer "F.Cu") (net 7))
 (segment (start 81 59.48) (end 87.52 59.48) (width 0.15) (layer "F.Cu") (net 7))
 (segment (start 77.68 62.8) (end 75.25 62.8) (width 0.15) (layer "F.Cu") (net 7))
 (segment (start 87.52 59.48) (end 90.81 62.77) (width 0.15) (layer "F.Cu") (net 7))
 (segment (start 111.54 49.62) (end 112.54 50.62) (width 0.15) (layer "F.Cu") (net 9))
 (segment (start 112.54 52.95) (end 113.86 54.27) (width 0.15) (layer "F.Cu") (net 9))
 (segment (start 109.66 49.62) (end 111.54 49.62) (width 0.15) (layer "F.Cu") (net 9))
 (segment (start 112.54 50.62) (end 112.54 52.95) (width 0.15) (layer "F.Cu") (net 9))
 (segment (start 107.38 57.28) (end 108.54 57.28) (width 0.3) (layer "F.Cu") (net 3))
 (via (at 108.54 57.28) (size 0.5) (drill 0.3) (layers "F.Cu" "B.Cu") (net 3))
 (segment (start 108.54 52.04) (end 106.8 50.3) (width 0.3) (layer "B.Cu") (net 3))
 (segment (start 113.86 46.65) (end 106.8 46.65) (width 0.3) (layer "B.Cu") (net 3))
 (segment (start 106.2 51.88995) (end 107.294975 50.794975) (width 0.3) (layer "B.Cu") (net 3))
 (segment (start 106.8 50.3) (end 104.98 52.12) (width 0.3) (layer "B.Cu") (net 3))
 (segment (start 108.54 57.28) (end 108.54 52.04) (width 0.3) (layer "B.Cu") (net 3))
 (segment (start 105.74 51.36) (end 106.8 50.3) (width 0.3) (layer "B.Cu") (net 3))
 (segment (start 106.8 46.65) (end 106.8 50.3) (width 0.3) (layer "B.Cu") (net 3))
 (segment (start 111.55 48.35) (end 112.39 49.19) (width 0.15) (layer "F.Cu") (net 10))
 (segment (start 109.66 48.35) (end 111.55 48.35) (width 0.15) (layer "F.Cu") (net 10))
 (segment (start 112.39 49.19) (end 113.86 49.19) (width 0.15) (layer "F.Cu") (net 10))
 (segment (start 84.12 47.67) (end 83.13 48.66) (width 0.15) (layer "F.Cu") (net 6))
 (segment (start 103.11 48.35) (end 102.43 47.67) (width 0.15) (layer "F.Cu") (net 6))
 (segment (start 102.43 47.67) (end 84.12 47.67) (width 0.15) (layer "F.Cu") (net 6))
 (segment (start 83.13 48.66) (end 81.055 48.66) (width 0.15) (layer "F.Cu") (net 6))
 (segment (start 81.055 48.66) (end 73.105 48.66) (width 0.15) (layer "F.Cu") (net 6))
 (segment (start 104.71 48.35) (end 103.11 48.35) (width 0.15) (layer "F.Cu") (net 6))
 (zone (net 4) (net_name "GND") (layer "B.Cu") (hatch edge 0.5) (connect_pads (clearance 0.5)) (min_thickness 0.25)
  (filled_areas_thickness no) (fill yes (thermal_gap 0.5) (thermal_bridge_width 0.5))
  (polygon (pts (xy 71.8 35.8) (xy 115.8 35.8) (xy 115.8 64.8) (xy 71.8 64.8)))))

